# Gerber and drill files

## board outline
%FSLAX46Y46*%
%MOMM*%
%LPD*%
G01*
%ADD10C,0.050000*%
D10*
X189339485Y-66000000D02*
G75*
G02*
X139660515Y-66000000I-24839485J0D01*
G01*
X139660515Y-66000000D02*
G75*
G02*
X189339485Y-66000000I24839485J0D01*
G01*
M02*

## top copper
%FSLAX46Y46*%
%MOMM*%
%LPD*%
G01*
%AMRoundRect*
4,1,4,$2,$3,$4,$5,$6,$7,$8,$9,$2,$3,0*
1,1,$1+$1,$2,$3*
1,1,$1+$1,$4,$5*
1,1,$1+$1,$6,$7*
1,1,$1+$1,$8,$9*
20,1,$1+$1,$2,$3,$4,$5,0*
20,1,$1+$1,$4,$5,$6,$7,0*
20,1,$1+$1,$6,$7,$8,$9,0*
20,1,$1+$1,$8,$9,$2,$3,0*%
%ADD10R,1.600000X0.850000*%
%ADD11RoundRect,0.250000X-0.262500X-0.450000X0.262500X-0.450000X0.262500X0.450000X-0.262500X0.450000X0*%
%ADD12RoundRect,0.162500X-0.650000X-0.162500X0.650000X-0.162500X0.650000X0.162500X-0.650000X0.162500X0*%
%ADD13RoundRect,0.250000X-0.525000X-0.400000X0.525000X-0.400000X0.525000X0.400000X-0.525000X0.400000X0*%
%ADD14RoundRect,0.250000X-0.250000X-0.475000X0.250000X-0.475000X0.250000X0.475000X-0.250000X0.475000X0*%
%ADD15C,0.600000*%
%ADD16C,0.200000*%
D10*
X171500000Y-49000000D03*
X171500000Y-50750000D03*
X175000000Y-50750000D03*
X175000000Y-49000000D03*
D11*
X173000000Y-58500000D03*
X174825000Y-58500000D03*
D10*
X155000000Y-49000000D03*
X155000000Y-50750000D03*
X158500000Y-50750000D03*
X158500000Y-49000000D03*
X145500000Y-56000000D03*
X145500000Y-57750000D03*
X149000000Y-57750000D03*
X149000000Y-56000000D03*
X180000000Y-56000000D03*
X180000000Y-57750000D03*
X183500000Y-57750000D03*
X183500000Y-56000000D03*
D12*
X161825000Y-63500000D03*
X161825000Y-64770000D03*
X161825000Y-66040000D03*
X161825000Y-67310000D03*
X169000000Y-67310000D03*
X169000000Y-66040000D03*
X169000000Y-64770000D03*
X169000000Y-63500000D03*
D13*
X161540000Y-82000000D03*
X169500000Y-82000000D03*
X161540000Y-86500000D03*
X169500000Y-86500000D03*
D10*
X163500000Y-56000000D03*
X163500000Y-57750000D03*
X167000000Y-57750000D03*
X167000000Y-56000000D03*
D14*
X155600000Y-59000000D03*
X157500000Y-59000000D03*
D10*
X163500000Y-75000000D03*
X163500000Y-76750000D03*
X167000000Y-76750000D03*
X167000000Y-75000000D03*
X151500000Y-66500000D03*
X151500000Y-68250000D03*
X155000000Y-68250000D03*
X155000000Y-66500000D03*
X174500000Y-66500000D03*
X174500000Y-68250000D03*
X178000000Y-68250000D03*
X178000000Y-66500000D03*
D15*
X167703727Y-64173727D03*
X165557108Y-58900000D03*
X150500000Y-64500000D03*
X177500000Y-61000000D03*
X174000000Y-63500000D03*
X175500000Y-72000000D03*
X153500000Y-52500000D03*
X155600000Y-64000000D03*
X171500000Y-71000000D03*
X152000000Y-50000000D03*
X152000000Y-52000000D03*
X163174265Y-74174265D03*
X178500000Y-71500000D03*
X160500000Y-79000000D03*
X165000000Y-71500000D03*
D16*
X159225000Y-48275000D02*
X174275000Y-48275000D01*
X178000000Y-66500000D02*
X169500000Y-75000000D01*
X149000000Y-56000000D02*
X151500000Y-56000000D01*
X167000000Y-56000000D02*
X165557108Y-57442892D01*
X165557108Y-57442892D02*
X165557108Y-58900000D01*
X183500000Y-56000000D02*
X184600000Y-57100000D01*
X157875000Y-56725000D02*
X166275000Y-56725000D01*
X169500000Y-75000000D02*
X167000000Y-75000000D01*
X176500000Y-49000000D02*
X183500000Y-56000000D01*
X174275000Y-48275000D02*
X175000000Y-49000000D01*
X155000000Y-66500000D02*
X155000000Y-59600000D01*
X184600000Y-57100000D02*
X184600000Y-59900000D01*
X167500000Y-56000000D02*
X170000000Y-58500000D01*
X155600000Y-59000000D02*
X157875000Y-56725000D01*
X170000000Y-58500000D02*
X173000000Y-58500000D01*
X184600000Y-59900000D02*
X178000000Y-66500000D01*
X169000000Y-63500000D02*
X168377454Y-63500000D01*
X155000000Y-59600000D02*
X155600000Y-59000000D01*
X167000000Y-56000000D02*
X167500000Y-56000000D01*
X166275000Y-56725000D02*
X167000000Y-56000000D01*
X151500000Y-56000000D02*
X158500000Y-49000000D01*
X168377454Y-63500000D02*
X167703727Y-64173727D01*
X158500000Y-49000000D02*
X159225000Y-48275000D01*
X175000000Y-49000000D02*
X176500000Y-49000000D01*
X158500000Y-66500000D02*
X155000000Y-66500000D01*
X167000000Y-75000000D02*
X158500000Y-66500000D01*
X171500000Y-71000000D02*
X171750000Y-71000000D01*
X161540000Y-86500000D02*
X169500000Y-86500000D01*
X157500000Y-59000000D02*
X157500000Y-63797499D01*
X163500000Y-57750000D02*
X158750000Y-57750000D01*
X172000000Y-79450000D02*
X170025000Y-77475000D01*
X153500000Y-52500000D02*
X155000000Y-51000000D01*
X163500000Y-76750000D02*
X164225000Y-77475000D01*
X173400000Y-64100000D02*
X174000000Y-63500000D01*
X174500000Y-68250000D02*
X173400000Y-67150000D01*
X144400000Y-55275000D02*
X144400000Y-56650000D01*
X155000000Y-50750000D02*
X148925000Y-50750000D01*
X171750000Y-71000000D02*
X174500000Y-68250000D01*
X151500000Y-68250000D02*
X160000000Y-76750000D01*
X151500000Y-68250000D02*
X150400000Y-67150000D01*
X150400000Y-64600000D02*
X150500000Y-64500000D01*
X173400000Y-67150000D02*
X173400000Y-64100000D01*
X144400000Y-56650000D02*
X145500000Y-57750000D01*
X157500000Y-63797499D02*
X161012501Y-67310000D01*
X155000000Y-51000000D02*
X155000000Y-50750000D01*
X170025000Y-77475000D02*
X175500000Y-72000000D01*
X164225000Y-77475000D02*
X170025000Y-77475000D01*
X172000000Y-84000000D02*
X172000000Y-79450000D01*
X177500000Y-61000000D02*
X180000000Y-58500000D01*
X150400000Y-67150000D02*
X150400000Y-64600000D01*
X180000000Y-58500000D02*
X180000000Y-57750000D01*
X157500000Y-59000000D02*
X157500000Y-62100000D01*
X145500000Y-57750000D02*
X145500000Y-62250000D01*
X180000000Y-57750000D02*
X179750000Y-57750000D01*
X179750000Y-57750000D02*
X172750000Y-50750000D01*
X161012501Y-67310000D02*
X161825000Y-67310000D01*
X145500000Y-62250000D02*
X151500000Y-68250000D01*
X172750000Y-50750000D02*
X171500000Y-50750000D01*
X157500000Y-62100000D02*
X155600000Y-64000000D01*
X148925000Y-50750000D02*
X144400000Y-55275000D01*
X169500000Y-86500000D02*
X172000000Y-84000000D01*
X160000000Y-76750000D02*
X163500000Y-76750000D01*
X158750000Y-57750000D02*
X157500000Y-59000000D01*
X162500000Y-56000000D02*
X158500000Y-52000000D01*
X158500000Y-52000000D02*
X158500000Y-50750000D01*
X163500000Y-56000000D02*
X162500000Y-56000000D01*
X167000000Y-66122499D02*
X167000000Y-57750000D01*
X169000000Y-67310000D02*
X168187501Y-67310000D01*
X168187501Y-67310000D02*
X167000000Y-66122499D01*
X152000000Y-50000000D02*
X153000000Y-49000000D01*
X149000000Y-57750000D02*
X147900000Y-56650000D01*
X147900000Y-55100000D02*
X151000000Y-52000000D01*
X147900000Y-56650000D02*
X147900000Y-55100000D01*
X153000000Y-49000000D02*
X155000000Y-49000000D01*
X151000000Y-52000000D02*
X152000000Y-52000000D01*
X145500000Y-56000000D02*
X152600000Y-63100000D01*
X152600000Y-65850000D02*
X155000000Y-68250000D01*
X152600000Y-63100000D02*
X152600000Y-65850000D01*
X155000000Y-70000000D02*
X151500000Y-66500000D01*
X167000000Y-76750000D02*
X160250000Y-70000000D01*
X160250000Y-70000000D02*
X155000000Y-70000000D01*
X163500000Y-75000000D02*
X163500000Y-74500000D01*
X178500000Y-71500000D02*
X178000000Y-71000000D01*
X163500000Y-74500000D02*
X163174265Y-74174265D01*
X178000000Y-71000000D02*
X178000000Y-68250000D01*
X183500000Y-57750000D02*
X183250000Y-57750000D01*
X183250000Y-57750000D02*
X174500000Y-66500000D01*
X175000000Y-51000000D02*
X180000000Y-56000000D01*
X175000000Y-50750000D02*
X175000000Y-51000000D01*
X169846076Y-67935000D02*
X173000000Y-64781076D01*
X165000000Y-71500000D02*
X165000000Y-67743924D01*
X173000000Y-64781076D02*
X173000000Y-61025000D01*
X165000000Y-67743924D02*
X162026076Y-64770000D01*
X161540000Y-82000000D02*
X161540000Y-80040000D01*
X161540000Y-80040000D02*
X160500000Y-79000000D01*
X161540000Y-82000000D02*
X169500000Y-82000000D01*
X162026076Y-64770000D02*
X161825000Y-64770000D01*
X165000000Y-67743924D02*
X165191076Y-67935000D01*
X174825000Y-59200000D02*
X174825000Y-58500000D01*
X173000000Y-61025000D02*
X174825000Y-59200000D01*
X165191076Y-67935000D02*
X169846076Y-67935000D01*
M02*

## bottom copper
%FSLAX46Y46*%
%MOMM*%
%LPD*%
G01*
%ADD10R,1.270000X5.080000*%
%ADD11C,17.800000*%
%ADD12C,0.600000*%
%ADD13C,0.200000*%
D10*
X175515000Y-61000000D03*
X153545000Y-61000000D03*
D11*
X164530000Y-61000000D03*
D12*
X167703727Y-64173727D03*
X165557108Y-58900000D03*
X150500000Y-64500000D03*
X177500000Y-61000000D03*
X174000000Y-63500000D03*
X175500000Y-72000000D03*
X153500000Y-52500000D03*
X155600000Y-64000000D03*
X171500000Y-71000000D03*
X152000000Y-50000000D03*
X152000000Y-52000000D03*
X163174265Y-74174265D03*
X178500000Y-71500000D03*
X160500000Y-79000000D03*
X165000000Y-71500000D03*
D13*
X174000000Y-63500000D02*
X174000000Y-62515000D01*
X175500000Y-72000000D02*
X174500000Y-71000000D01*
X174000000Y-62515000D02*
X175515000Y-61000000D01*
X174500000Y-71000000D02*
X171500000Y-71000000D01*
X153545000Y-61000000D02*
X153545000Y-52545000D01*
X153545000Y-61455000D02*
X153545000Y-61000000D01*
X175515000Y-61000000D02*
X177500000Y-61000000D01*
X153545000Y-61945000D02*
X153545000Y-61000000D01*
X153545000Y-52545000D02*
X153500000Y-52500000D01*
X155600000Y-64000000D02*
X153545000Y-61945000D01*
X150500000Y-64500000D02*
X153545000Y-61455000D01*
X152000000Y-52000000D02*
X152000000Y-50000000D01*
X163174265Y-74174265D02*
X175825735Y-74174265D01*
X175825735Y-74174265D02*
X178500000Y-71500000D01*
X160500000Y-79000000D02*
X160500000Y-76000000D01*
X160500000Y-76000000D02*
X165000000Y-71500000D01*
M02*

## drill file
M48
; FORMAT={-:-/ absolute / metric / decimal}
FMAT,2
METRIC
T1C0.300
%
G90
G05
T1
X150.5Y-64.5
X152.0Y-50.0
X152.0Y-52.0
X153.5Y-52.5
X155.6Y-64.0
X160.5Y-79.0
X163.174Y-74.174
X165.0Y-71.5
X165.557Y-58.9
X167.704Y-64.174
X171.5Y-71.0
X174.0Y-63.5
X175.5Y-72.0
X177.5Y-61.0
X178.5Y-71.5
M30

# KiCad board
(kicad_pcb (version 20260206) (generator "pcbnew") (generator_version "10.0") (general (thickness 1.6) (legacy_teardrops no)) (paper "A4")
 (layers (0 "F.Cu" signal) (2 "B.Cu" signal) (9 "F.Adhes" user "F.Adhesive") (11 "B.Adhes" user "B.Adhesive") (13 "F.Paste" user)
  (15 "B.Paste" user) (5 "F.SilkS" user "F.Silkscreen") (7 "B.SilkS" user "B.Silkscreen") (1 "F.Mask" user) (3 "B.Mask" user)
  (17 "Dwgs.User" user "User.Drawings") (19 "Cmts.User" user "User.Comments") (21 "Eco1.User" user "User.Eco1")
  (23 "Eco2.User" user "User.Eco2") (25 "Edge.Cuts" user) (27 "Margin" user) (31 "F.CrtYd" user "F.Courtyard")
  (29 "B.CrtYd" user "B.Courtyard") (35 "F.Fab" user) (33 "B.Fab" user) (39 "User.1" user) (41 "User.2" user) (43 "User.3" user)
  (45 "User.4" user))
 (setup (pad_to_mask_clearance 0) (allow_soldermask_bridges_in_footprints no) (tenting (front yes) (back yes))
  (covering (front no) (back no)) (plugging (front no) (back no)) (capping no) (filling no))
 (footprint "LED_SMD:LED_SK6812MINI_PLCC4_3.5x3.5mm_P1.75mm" (layer "F.Cu") (at 173.25 49.875)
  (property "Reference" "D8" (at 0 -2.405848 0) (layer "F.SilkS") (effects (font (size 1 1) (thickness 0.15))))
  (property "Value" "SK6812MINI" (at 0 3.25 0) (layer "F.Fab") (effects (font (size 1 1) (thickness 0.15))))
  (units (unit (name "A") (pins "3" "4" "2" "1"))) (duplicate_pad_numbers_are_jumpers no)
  (pad "1" smd rect (at -1.75 -0.875) (size 1.6 0.85) (layers "F.Cu" "F.Mask" "F.Paste") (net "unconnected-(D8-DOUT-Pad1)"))
  (pad "2" smd rect (at -1.75 0.875) (size 1.6 0.85) (layers "F.Cu" "F.Mask" "F.Paste") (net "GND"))
  (pad "3" smd rect (at 1.75 0.875) (size 1.6 0.85) (layers "F.Cu" "F.Mask" "F.Paste") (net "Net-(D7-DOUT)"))
  (pad "4" smd rect (at 1.75 -0.875) (size 1.6 0.85) (layers "F.Cu" "F.Mask" "F.Paste") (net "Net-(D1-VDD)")))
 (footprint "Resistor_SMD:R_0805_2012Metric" (layer "F.Cu") (at 173.9125 58.5)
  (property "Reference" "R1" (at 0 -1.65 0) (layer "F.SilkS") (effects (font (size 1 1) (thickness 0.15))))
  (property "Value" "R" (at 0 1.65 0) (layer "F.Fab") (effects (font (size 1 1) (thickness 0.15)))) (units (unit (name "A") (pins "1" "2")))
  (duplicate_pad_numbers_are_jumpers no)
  (pad "1" smd roundrect (at -0.9125 0) (size 1.025 1.4) (layers "F.Cu" "F.Mask" "F.Paste") (roundrect_rratio 0.243902) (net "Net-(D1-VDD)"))
  (pad "2" smd roundrect (at 0.9125 0) (size 1.025 1.4) (layers "F.Cu" "F.Mask" "F.Paste") (roundrect_rratio 0.243902)
   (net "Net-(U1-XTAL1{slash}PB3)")))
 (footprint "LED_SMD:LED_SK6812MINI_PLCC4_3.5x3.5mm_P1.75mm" (layer "F.Cu") (at 156.75 49.875)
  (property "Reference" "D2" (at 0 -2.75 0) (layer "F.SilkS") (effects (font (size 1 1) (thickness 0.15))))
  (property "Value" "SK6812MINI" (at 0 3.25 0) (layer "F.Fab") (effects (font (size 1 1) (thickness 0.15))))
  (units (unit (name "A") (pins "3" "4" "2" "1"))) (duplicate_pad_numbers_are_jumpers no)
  (pad "1" smd rect (at -1.75 -0.875) (size 1.6 0.85) (layers "F.Cu" "F.Mask" "F.Paste") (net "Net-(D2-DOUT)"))
  (pad "2" smd rect (at -1.75 0.875) (size 1.6 0.85) (layers "F.Cu" "F.Mask" "F.Paste") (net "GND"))
  (pad "3" smd rect (at 1.75 0.875) (size 1.6 0.85) (layers "F.Cu" "F.Mask" "F.Paste") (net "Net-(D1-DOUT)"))
  (pad "4" smd rect (at 1.75 -0.875) (size 1.6 0.85) (layers "F.Cu" "F.Mask" "F.Paste") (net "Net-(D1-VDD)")))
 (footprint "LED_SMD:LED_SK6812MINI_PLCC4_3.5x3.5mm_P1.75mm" (layer "F.Cu") (at 147.25 56.875)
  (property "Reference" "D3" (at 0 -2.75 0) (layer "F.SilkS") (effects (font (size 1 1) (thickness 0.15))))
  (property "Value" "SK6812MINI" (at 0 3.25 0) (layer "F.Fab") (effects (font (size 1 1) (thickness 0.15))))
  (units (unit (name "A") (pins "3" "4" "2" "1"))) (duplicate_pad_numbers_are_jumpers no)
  (pad "1" smd rect (at -1.75 -0.875) (size 1.6 0.85) (layers "F.Cu" "F.Mask" "F.Paste") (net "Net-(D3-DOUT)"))
  (pad "2" smd rect (at -1.75 0.875) (size 1.6 0.85) (layers "F.Cu" "F.Mask" "F.Paste") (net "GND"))
  (pad "3" smd rect (at 1.75 0.875) (size 1.6 0.85) (layers "F.Cu" "F.Mask" "F.Paste") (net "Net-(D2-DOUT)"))
  (pad "4" smd rect (at 1.75 -0.875) (size 1.6 0.85) (layers "F.Cu" "F.Mask" "F.Paste") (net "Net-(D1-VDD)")))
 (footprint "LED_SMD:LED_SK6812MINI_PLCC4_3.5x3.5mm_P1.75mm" (layer "F.Cu") (at 181.75 56.875)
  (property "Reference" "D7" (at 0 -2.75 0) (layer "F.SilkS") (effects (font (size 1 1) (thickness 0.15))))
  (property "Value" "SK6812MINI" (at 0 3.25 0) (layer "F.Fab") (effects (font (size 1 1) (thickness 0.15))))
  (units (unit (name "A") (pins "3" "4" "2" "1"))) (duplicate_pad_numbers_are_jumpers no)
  (pad "1" smd rect (at -1.75 -0.875) (size 1.6 0.85) (layers "F.Cu" "F.Mask" "F.Paste") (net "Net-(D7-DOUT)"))
  (pad "2" smd rect (at -1.75 0.875) (size 1.6 0.85) (layers "F.Cu" "F.Mask" "F.Paste") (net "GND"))
  (pad "3" smd rect (at 1.75 0.875) (size 1.6 0.85) (layers "F.Cu" "F.Mask" "F.Paste") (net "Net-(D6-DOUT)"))
  (pad "4" smd rect (at 1.75 -0.875) (size 1.6 0.85) (layers "F.Cu" "F.Mask" "F.Paste") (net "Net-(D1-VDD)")))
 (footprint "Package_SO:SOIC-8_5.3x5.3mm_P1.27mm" (layer "F.Cu") (at 165.4125 65.405)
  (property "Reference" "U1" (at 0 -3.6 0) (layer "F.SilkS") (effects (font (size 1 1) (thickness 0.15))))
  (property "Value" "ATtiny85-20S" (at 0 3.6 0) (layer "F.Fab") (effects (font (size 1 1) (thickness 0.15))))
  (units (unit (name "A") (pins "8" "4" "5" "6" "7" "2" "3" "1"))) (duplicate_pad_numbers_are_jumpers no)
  (pad "1" smd roundrect (at -3.5875 -1.905) (size 1.625 0.65) (layers "F.Cu" "F.Mask" "F.Paste") (roundrect_rratio 0.25)
   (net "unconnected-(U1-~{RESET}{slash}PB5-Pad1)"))
  (pad "2" smd roundrect (at -3.5875 -0.635) (size 1.625 0.65) (layers "F.Cu" "F.Mask" "F.Paste") (roundrect_rratio 0.25)
   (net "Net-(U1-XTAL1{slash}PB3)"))
  (pad "3" smd roundrect (at -3.5875 0.635) (size 1.625 0.65) (layers "F.Cu" "F.Mask" "F.Paste") (roundrect_rratio 0.25)
   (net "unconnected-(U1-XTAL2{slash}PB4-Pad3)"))
  (pad "4" smd roundrect (at -3.5875 1.905) (size 1.625 0.65) (layers "F.Cu" "F.Mask" "F.Paste") (roundrect_rratio 0.25) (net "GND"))
  (pad "5" smd roundrect (at 3.5875 1.905) (size 1.625 0.65) (layers "F.Cu" "F.Mask" "F.Paste") (roundrect_rratio 0.25) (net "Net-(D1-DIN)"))
  (pad "6" smd roundrect (at 3.5875 0.635) (size 1.625 0.65) (layers "F.Cu" "F.Mask" "F.Paste") (roundrect_rratio 0.25)
   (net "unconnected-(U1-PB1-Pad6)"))
  (pad "7" smd roundrect (at 3.5875 -0.635) (size 1.625 0.65) (layers "F.Cu" "F.Mask" "F.Paste") (roundrect_rratio 0.25)
   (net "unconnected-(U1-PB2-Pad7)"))
  (pad "8" smd roundrect (at 3.5875 -1.905) (size 1.625 0.65) (layers "F.Cu" "F.Mask" "F.Paste") (roundrect_rratio 0.25)
   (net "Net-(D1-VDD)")))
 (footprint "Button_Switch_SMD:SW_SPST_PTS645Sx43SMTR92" (layer "F.Cu") (at 165.52 84.25)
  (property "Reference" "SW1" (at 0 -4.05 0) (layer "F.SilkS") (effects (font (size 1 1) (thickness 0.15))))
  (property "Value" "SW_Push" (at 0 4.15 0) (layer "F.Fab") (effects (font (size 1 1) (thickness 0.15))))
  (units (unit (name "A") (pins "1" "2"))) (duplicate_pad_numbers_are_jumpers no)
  (pad "1" smd roundrect (at -3.98 -2.25) (size 1.55 1.3) (layers "F.Cu" "F.Mask" "F.Paste") (roundrect_rratio 0.1923076923)
   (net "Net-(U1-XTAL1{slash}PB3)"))
  (pad "1" smd roundrect (at 3.98 -2.25) (size 1.55 1.3) (layers "F.Cu" "F.Mask" "F.Paste") (roundrect_rratio 0.1923076923)
   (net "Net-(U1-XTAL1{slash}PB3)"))
  (pad "2" smd roundrect (at -3.98 2.25) (size 1.55 1.3) (layers "F.Cu" "F.Mask" "F.Paste") (roundrect_rratio 0.1923076923) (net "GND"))
  (pad "2" smd roundrect (at 3.98 2.25) (size 1.55 1.3) (layers "F.Cu" "F.Mask" "F.Paste") (roundrect_rratio 0.1923076923) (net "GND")))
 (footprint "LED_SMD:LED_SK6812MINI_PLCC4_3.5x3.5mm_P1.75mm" (layer "F.Cu") (at 165.25 56.875)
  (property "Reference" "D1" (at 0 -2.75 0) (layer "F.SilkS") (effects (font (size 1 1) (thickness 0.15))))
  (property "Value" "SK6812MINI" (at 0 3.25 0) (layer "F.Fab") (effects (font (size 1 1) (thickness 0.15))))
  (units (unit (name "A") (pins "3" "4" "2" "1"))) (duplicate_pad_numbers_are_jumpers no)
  (pad "1" smd rect (at -1.75 -0.875) (size 1.6 0.85) (layers "F.Cu" "F.Mask" "F.Paste") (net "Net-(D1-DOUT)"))
  (pad "2" smd rect (at -1.75 0.875) (size 1.6 0.85) (layers "F.Cu" "F.Mask" "F.Paste") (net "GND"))
  (pad "3" smd rect (at 1.75 0.875) (size 1.6 0.85) (layers "F.Cu" "F.Mask" "F.Paste") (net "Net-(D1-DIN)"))
  (pad "4" smd rect (at 1.75 -0.875) (size 1.6 0.85) (layers "F.Cu" "F.Mask" "F.Paste") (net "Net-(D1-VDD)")))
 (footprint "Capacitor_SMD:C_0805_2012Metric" (layer "F.Cu") (at 156.55 59)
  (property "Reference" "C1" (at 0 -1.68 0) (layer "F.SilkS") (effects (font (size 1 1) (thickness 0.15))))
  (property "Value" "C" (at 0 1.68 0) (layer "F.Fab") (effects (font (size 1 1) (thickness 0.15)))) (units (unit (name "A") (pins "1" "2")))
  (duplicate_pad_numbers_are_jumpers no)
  (pad "1" smd roundrect (at -0.95 0) (size 1 1.45) (layers "F.Cu" "F.Mask" "F.Paste") (roundrect_rratio 0.25) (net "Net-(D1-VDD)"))
  (pad "2" smd roundrect (at 0.95 0) (size 1 1.45) (layers "F.Cu" "F.Mask" "F.Paste") (roundrect_rratio 0.25) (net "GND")))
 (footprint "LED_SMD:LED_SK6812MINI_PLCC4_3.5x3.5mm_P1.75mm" (layer "F.Cu") (at 165.25 75.875)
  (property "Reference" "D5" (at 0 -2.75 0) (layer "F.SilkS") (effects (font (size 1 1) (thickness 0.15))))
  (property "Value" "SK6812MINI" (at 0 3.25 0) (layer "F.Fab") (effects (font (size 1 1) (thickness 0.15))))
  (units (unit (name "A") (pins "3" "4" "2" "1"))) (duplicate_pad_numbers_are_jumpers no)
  (pad "1" smd rect (at -1.75 -0.875) (size 1.6 0.85) (layers "F.Cu" "F.Mask" "F.Paste") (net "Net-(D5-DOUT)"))
  (pad "2" smd rect (at -1.75 0.875) (size 1.6 0.85) (layers "F.Cu" "F.Mask" "F.Paste") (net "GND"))
  (pad "3" smd rect (at 1.75 0.875) (size 1.6 0.85) (layers "F.Cu" "F.Mask" "F.Paste") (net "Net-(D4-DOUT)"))
  (pad "4" smd rect (at 1.75 -0.875) (size 1.6 0.85) (layers "F.Cu" "F.Mask" "F.Paste") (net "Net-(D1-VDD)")))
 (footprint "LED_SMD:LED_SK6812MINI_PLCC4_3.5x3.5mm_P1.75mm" (layer "F.Cu") (at 153.25 67.375)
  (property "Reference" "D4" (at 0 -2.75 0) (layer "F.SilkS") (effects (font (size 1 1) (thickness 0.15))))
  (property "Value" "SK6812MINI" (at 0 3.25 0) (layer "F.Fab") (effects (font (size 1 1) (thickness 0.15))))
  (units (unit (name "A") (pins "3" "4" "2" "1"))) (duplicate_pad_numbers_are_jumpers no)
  (pad "1" smd rect (at -1.75 -0.875) (size 1.6 0.85) (layers "F.Cu" "F.Mask" "F.Paste") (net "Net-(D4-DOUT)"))
  (pad "2" smd rect (at -1.75 0.875) (size 1.6 0.85) (layers "F.Cu" "F.Mask" "F.Paste") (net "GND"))
  (pad "3" smd rect (at 1.75 0.875) (size 1.6 0.85) (layers "F.Cu" "F.Mask" "F.Paste") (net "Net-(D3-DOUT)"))
  (pad "4" smd rect (at 1.75 -0.875) (size 1.6 0.85) (layers "F.Cu" "F.Mask" "F.Paste") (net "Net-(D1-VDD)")))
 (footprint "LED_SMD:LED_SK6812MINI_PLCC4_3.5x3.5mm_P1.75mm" (layer "F.Cu") (at 176.25 67.375)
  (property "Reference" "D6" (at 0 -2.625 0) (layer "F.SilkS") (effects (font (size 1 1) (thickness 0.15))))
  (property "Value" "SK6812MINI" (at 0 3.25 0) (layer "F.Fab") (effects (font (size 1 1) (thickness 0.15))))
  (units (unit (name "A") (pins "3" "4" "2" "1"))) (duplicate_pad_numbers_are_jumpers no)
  (pad "1" smd rect (at -1.75 -0.875) (size 1.6 0.85) (layers "F.Cu" "F.Mask" "F.Paste") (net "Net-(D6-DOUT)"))
  (pad "2" smd rect (at -1.75 0.875) (size 1.6 0.85) (layers "F.Cu" "F.Mask" "F.Paste") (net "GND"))
  (pad "3" smd rect (at 1.75 0.875) (size 1.6 0.85) (layers "F.Cu" "F.Mask" "F.Paste") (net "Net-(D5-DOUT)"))
  (pad "4" smd rect (at 1.75 -0.875) (size 1.6 0.85) (layers "F.Cu" "F.Mask" "F.Paste") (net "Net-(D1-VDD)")))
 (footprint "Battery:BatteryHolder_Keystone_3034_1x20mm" (layer "B.Cu") (at 164.53 61 180)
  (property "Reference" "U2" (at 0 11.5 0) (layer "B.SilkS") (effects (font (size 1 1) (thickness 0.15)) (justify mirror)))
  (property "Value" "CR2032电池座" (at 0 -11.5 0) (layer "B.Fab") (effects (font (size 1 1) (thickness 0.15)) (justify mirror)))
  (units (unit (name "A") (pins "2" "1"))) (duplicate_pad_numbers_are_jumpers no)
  (pad "1" smd rect (at -10.985 0 180) (size 1.27 5.08) (layers "B.Cu" "B.Mask" "B.Paste") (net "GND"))
  (pad "1" smd rect (at 10.985 0 180) (size 1.27 5.08) (layers "B.Cu" "B.Mask" "B.Paste") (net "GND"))
  (pad "2" smd circle (at 0 0 180) (size 17.8 17.8) (layers "B.Cu" "B.Mask") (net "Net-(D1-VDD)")))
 (gr_circle (center 164.5 66) (end 180.5 85) (stroke (width 0.05) (type default)) (fill no) (layer "Edge.Cuts"))
 (segment (start 159.225 48.275) (end 174.275 48.275) (width 0.2) (layer "F.Cu") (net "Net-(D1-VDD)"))
 (segment (start 178 66.5) (end 169.5 75) (width 0.2) (layer "F.Cu") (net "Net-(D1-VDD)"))
 (segment (start 149 56) (end 151.5 56) (width 0.2) (layer "F.Cu") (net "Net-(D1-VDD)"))
 (segment (start 167 56) (end 165.557108 57.442892) (width 0.2) (layer "F.Cu") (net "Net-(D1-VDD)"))
 (segment (start 165.557108 57.442892) (end 165.557108 58.9) (width 0.2) (layer "F.Cu") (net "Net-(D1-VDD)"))
 (segment (start 183.5 56) (end 184.6 57.1) (width 0.2) (layer "F.Cu") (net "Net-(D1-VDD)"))
 (segment (start 157.875 56.725) (end 166.275 56.725) (width 0.2) (layer "F.Cu") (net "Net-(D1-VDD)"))
 (segment (start 169.5 75) (end 167 75) (width 0.2) (layer "F.Cu") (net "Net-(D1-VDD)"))
 (segment (start 176.5 49) (end 183.5 56) (width 0.2) (layer "F.Cu") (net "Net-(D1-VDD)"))
 (segment (start 174.275 48.275) (end 175 49) (width 0.2) (layer "F.Cu") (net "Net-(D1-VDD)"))
 (segment (start 155 66.5) (end 155 59.6) (width 0.2) (layer "F.Cu") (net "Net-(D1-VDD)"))
 (segment (start 184.6 57.1) (end 184.6 59.9) (width 0.2) (layer "F.Cu") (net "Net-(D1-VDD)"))
 (segment (start 167.5 56) (end 170 58.5) (width 0.2) (layer "F.Cu") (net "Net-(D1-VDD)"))
 (segment (start 155.6 59) (end 157.875 56.725) (width 0.2) (layer "F.Cu") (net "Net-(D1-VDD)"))
 (segment (start 170 58.5) (end 173 58.5) (width 0.2) (layer "F.Cu") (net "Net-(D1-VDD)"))
 (segment (start 184.6 59.9) (end 178 66.5) (width 0.2) (layer "F.Cu") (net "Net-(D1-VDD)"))
 (segment (start 169 63.5) (end 168.377454 63.5) (width 0.2) (layer "F.Cu") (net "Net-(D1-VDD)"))
 (segment (start 155 59.6) (end 155.6 59) (width 0.2) (layer "F.Cu") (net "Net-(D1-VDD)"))
 (segment (start 167 56) (end 167.5 56) (width 0.2) (layer "F.Cu") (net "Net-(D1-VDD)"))
 (segment (start 166.275 56.725) (end 167 56) (width 0.2) (layer "F.Cu") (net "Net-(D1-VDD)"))
 (segment (start 151.5 56) (end 158.5 49) (width 0.2) (layer "F.Cu") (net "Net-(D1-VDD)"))
 (segment (start 168.377454 63.5) (end 167.703727 64.173727) (width 0.2) (layer "F.Cu") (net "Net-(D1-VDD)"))
 (segment (start 158.5 49) (end 159.225 48.275) (width 0.2) (layer "F.Cu") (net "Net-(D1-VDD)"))
 (segment (start 175 49) (end 176.5 49) (width 0.2) (layer "F.Cu") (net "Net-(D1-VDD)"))
 (segment (start 158.5 66.5) (end 155 66.5) (width 0.2) (layer "F.Cu") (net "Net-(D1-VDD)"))
 (segment (start 167 75) (end 158.5 66.5) (width 0.2) (layer "F.Cu") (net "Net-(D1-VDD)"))
 (via (at 167.703727 64.173727) (size 0.6) (drill 0.3) (layers "F.Cu" "B.Cu") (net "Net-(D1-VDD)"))
 (via (at 165.557108 58.9) (size 0.6) (drill 0.3) (layers "F.Cu" "B.Cu") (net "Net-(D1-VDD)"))
 (segment (start 171.5 71) (end 171.75 71) (width 0.2) (layer "F.Cu") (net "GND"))
 (segment (start 161.54 86.5) (end 169.5 86.5) (width 0.2) (layer "F.Cu") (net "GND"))
 (segment (start 157.5 59) (end 157.5 63.797499) (width 0.2) (layer "F.Cu") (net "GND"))
 (segment (start 163.5 57.75) (end 158.75 57.75) (width 0.2) (layer "F.Cu") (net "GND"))
 (segment (start 172 79.45) (end 170.025 77.475) (width 0.2) (layer "F.Cu") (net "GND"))
 (segment (start 153.5 52.5) (end 155 51) (width 0.2) (layer "F.Cu") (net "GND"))
 (segment (start 163.5 76.75) (end 164.225 77.475) (width 0.2) (layer "F.Cu") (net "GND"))
 (segment (start 173.4 64.1) (end 174 63.5) (width 0.2) (layer "F.Cu") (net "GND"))
 (segment (start 174.5 68.25) (end 173.4 67.15) (width 0.2) (layer "F.Cu") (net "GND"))
 (segment (start 144.4 55.275) (end 144.4 56.65) (width 0.2) (layer "F.Cu") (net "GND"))
 (segment (start 155 50.75) (end 148.925 50.75) (width 0.2) (layer "F.Cu") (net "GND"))
 (segment (start 171.75 71) (end 174.5 68.25) (width 0.2) (layer "F.Cu") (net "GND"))
 (segment (start 151.5 68.25) (end 160 76.75) (width 0.2) (layer "F.Cu") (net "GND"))
 (segment (start 151.5 68.25) (end 150.4 67.15) (width 0.2) (layer "F.Cu") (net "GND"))
 (segment (start 150.4 64.6) (end 150.5 64.5) (width 0.2) (layer "F.Cu") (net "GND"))
 (segment (start 173.4 67.15) (end 173.4 64.1) (width 0.2) (layer "F.Cu") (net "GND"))
 (segment (start 144.4 56.65) (end 145.5 57.75) (width 0.2) (layer "F.Cu") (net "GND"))
 (segment (start 157.5 63.797499) (end 161.012501 67.31) (width 0.2) (layer "F.Cu") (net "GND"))
 (segment (start 155 51) (end 155 50.75) (width 0.2) (layer "F.Cu") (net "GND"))
 (segment (start 170.025 77.475) (end 175.5 72) (width 0.2) (layer "F.Cu") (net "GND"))
 (segment (start 164.225 77.475) (end 170.025 77.475) (width 0.2) (layer "F.Cu") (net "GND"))
 (segment (start 172 84) (end 172 79.45) (width 0.2) (layer "F.Cu") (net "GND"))
 (segment (start 177.5 61) (end 180 58.5) (width 0.2) (layer "F.Cu") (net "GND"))
 (segment (start 150.4 67.15) (end 150.4 64.6) (width 0.2) (layer "F.Cu") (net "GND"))
 (segment (start 180 58.5) (end 180 57.75) (width 0.2) (layer "F.Cu") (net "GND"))
 (segment (start 157.5 59) (end 157.5 62.1) (width 0.2) (layer "F.Cu") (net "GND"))
 (segment (start 145.5 57.75) (end 145.5 62.25) (width 0.2) (layer "F.Cu") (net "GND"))
 (segment (start 180 57.75) (end 179.75 57.75) (width 0.2) (layer "F.Cu") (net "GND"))
 (segment (start 179.75 57.75) (end 172.75 50.75) (width 0.2) (layer "F.Cu") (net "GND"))
 (segment (start 161.012501 67.31) (end 161.825 67.31) (width 0.2) (layer "F.Cu") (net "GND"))
 (segment (start 145.5 62.25) (end 151.5 68.25) (width 0.2) (layer "F.Cu") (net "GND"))
 (segment (start 172.75 50.75) (end 171.5 50.75) (width 0.2) (layer "F.Cu") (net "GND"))
 (segment (start 157.5 62.1) (end 155.6 64) (width 0.2) (layer "F.Cu") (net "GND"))
 (segment (start 148.925 50.75) (end 144.4 55.275) (width 0.2) (layer "F.Cu") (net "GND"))
 (segment (start 169.5 86.5) (end 172 84) (width 0.2) (layer "F.Cu") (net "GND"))
 (segment (start 160 76.75) (end 163.5 76.75) (width 0.2) (layer "F.Cu") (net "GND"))
 (segment (start 158.75 57.75) (end 157.5 59) (width 0.2) (layer "F.Cu") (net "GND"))
 (via (at 150.5 64.5) (size 0.6) (drill 0.3) (layers "F.Cu" "B.Cu") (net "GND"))
 (via (at 177.5 61) (size 0.6) (drill 0.3) (layers "F.Cu" "B.Cu") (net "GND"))
 (via (at 174 63.5) (size 0.6) (drill 0.3) (layers "F.Cu" "B.Cu") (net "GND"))
 (via (at 175.5 72) (size 0.6) (drill 0.3) (layers "F.Cu" "B.Cu") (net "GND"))
 (via (at 153.5 52.5) (size 0.6) (drill 0.3) (layers "F.Cu" "B.Cu") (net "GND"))
 (via (at 155.6 64) (size 0.6) (drill 0.3) (layers "F.Cu" "B.Cu") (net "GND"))
 (via (at 171.5 71) (size 0.6) (drill 0.3) (layers "F.Cu" "B.Cu") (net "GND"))
 (segment (start 174 63.5) (end 174 62.515) (width 0.2) (layer "B.Cu") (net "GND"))
 (segment (start 175.5 72) (end 174.5 71) (width 0.2) (layer "B.Cu") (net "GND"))
 (segment (start 174 62.515) (end 175.515 61) (width 0.2) (layer "B.Cu") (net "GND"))
 (segment (start 174.5 71) (end 171.5 71) (width 0.2) (layer "B.Cu") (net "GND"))
 (segment (start 153.545 61) (end 153.545 52.545) (width 0.2) (layer "B.Cu") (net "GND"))
 (segment (start 153.545 61.455) (end 153.545 61) (width 0.2) (layer "B.Cu") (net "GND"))
 (segment (start 175.515 61) (end 177.5 61) (width 0.2) (layer "B.Cu") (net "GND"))
 (segment (start 153.545 61.945) (end 153.545 61) (width 0.2) (layer "B.Cu") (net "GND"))
 (segment (start 153.545 52.545) (end 153.5 52.5) (width 0.2) (layer "B.Cu") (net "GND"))
 (segment (start 155.6 64) (end 153.545 61.945) (width 0.2) (layer "B.Cu") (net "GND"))
 (segment (start 150.5 64.5) (end 153.545 61.455) (width 0.2) (layer "B.Cu") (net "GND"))
 (segment (start 162.5 56) (end 158.5 52) (width 0.2) (layer "F.Cu") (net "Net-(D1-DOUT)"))
 (segment (start 158.5 52) (end 158.5 50.75) (width 0.2) (layer "F.Cu") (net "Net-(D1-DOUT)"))
 (segment (start 163.5 56) (end 162.5 56) (width 0.2) (layer "F.Cu") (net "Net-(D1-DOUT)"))
 (segment (start 167 66.122499) (end 167 57.75) (width 0.2) (layer "F.Cu") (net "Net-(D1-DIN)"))
 (segment (start 169 67.31) (end 168.187501 67.31) (width 0.2) (layer "F.Cu") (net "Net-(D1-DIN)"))
 (segment (start 168.187501 67.31) (end 167 66.122499) (width 0.2) (layer "F.Cu") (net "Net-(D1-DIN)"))
 (segment (start 152 50) (end 153 49) (width 0.2) (layer "F.Cu") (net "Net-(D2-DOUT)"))
 (segment (start 149 57.75) (end 147.9 56.65) (width 0.2) (layer "F.Cu") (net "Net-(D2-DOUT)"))
 (segment (start 147.9 55.1) (end 151 52) (width 0.2) (layer "F.Cu") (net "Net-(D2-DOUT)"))
 (segment (start 147.9 56.65) (end 147.9 55.1) (width 0.2) (layer "F.Cu") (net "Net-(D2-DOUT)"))
 (segment (start 153 49) (end 155 49) (width 0.2) (layer "F.Cu") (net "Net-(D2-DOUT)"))
 (segment (start 151 52) (end 152 52) (width 0.2) (layer "F.Cu") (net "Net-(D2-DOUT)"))
 (via (at 152 50) (size 0.6) (drill 0.3) (layers "F.Cu" "B.Cu") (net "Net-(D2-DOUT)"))
 (via (at 152 52) (size 0.6) (drill 0.3) (layers "F.Cu" "B.Cu") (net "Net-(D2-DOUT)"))
 (segment (start 152 52) (end 152 50) (width 0.2) (layer "B.Cu") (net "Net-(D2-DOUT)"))
 (segment (start 145.5 56) (end 152.6 63.1) (width 0.2) (layer "F.Cu") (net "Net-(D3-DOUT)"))
 (segment (start 152.6 65.85) (end 155 68.25) (width 0.2) (layer "F.Cu") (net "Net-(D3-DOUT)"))
 (segment (start 152.6 63.1) (end 152.6 65.85) (width 0.2) (layer "F.Cu") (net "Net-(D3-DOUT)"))
 (segment (start 155 70) (end 151.5 66.5) (width 0.2) (layer "F.Cu") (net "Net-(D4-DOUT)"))
 (segment (start 167 76.75) (end 160.25 70) (width 0.2) (layer "F.Cu") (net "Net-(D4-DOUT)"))
 (segment (start 160.25 70) (end 155 70) (width 0.2) (layer "F.Cu") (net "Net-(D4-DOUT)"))
 (segment (start 163.5 75) (end 163.5 74.5) (width 0.2) (layer "F.Cu") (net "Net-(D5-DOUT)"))
 (segment (start 178.5 71.5) (end 178 71) (width 0.2) (layer "F.Cu") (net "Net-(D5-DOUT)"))
 (segment (start 163.5 74.5) (end 163.174265 74.174265) (width 0.2) (layer "F.Cu") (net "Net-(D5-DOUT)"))
 (segment (start 178 71) (end 178 68.25) (width 0.2) (layer "F.Cu") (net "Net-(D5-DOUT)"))
 (via (at 163.174265 74.174265) (size 0.6) (drill 0.3) (layers "F.Cu" "B.Cu") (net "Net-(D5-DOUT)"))
 (via (at 178.5 71.5) (size 0.6) (drill 0.3) (layers "F.Cu" "B.Cu") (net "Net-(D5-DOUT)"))
 (segment (start 163.174265 74.174265) (end 175.825735 74.174265) (width 0.2) (layer "B.Cu") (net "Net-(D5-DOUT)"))
 (segment (start 175.825735 74.174265) (end 178.5 71.5) (width 0.2) (layer "B.Cu") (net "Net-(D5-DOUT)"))
 (segment (start 183.5 57.75) (end 183.25 57.75) (width 0.2) (layer "F.Cu") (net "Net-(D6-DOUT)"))
 (segment (start 183.25 57.75) (end 174.5 66.5) (width 0.2) (layer "F.Cu") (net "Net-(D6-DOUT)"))
 (segment (start 175 51) (end 180 56) (width 0.2) (layer "F.Cu") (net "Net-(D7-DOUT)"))
 (segment (start 175 50.75) (end 175 51) (width 0.2) (layer "F.Cu") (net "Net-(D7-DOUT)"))
 (segment (start 169.846076 67.935) (end 173 64.781076) (width 0.2) (layer "F.Cu") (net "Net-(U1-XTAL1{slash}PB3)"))
 (segment (start 165 71.5) (end 165 67.743924) (width 0.2) (layer "F.Cu") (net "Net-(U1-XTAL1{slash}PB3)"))
 (segment (start 173 64.781076) (end 173 61.025) (width 0.2) (layer "F.Cu") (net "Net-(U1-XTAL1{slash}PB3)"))
 (segment (start 165 67.743924) (end 162.026076 64.77) (width 0.2) (layer "F.Cu") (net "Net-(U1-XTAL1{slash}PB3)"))
 (segment (start 161.54 82) (end 161.54 80.04) (width 0.2) (layer "F.Cu") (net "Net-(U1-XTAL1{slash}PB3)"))
 (segment (start 161.54 80.04) (end 160.5 79) (width 0.2) (layer "F.Cu") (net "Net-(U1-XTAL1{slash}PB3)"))
 (segment (start 161.54 82) (end 169.5 82) (width 0.2) (layer "F.Cu") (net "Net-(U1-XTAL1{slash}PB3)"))
 (segment (start 162.026076 64.77) (end 161.825 64.77) (width 0.2) (layer "F.Cu") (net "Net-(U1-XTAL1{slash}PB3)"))
 (segment (start 165 67.743924) (end 165.191076 67.935) (width 0.2) (layer "F.Cu") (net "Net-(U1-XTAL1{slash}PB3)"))
 (segment (start 174.825 59.2) (end 174.825 58.5) (width 0.2) (layer "F.Cu") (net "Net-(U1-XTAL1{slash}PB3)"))
 (segment (start 173 61.025) (end 174.825 59.2) (width 0.2) (layer "F.Cu") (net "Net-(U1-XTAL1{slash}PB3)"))
 (segment (start 165.191076 67.935) (end 169.846076 67.935) (width 0.2) (layer "F.Cu") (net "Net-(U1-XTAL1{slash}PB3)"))
 (via (at 160.5 79) (size 0.6) (drill 0.3) (layers "F.Cu" "B.Cu") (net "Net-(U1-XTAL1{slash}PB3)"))
 (via (at 165 71.5) (size 0.6) (drill 0.3) (layers "F.Cu" "B.Cu") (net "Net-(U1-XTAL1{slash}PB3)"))
 (segment (start 160.5 79) (end 160.5 76) (width 0.2) (layer "B.Cu") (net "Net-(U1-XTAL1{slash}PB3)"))
 (segment (start 160.5 76) (end 165 71.5) (width 0.2) (layer "B.Cu") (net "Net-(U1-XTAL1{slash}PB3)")))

